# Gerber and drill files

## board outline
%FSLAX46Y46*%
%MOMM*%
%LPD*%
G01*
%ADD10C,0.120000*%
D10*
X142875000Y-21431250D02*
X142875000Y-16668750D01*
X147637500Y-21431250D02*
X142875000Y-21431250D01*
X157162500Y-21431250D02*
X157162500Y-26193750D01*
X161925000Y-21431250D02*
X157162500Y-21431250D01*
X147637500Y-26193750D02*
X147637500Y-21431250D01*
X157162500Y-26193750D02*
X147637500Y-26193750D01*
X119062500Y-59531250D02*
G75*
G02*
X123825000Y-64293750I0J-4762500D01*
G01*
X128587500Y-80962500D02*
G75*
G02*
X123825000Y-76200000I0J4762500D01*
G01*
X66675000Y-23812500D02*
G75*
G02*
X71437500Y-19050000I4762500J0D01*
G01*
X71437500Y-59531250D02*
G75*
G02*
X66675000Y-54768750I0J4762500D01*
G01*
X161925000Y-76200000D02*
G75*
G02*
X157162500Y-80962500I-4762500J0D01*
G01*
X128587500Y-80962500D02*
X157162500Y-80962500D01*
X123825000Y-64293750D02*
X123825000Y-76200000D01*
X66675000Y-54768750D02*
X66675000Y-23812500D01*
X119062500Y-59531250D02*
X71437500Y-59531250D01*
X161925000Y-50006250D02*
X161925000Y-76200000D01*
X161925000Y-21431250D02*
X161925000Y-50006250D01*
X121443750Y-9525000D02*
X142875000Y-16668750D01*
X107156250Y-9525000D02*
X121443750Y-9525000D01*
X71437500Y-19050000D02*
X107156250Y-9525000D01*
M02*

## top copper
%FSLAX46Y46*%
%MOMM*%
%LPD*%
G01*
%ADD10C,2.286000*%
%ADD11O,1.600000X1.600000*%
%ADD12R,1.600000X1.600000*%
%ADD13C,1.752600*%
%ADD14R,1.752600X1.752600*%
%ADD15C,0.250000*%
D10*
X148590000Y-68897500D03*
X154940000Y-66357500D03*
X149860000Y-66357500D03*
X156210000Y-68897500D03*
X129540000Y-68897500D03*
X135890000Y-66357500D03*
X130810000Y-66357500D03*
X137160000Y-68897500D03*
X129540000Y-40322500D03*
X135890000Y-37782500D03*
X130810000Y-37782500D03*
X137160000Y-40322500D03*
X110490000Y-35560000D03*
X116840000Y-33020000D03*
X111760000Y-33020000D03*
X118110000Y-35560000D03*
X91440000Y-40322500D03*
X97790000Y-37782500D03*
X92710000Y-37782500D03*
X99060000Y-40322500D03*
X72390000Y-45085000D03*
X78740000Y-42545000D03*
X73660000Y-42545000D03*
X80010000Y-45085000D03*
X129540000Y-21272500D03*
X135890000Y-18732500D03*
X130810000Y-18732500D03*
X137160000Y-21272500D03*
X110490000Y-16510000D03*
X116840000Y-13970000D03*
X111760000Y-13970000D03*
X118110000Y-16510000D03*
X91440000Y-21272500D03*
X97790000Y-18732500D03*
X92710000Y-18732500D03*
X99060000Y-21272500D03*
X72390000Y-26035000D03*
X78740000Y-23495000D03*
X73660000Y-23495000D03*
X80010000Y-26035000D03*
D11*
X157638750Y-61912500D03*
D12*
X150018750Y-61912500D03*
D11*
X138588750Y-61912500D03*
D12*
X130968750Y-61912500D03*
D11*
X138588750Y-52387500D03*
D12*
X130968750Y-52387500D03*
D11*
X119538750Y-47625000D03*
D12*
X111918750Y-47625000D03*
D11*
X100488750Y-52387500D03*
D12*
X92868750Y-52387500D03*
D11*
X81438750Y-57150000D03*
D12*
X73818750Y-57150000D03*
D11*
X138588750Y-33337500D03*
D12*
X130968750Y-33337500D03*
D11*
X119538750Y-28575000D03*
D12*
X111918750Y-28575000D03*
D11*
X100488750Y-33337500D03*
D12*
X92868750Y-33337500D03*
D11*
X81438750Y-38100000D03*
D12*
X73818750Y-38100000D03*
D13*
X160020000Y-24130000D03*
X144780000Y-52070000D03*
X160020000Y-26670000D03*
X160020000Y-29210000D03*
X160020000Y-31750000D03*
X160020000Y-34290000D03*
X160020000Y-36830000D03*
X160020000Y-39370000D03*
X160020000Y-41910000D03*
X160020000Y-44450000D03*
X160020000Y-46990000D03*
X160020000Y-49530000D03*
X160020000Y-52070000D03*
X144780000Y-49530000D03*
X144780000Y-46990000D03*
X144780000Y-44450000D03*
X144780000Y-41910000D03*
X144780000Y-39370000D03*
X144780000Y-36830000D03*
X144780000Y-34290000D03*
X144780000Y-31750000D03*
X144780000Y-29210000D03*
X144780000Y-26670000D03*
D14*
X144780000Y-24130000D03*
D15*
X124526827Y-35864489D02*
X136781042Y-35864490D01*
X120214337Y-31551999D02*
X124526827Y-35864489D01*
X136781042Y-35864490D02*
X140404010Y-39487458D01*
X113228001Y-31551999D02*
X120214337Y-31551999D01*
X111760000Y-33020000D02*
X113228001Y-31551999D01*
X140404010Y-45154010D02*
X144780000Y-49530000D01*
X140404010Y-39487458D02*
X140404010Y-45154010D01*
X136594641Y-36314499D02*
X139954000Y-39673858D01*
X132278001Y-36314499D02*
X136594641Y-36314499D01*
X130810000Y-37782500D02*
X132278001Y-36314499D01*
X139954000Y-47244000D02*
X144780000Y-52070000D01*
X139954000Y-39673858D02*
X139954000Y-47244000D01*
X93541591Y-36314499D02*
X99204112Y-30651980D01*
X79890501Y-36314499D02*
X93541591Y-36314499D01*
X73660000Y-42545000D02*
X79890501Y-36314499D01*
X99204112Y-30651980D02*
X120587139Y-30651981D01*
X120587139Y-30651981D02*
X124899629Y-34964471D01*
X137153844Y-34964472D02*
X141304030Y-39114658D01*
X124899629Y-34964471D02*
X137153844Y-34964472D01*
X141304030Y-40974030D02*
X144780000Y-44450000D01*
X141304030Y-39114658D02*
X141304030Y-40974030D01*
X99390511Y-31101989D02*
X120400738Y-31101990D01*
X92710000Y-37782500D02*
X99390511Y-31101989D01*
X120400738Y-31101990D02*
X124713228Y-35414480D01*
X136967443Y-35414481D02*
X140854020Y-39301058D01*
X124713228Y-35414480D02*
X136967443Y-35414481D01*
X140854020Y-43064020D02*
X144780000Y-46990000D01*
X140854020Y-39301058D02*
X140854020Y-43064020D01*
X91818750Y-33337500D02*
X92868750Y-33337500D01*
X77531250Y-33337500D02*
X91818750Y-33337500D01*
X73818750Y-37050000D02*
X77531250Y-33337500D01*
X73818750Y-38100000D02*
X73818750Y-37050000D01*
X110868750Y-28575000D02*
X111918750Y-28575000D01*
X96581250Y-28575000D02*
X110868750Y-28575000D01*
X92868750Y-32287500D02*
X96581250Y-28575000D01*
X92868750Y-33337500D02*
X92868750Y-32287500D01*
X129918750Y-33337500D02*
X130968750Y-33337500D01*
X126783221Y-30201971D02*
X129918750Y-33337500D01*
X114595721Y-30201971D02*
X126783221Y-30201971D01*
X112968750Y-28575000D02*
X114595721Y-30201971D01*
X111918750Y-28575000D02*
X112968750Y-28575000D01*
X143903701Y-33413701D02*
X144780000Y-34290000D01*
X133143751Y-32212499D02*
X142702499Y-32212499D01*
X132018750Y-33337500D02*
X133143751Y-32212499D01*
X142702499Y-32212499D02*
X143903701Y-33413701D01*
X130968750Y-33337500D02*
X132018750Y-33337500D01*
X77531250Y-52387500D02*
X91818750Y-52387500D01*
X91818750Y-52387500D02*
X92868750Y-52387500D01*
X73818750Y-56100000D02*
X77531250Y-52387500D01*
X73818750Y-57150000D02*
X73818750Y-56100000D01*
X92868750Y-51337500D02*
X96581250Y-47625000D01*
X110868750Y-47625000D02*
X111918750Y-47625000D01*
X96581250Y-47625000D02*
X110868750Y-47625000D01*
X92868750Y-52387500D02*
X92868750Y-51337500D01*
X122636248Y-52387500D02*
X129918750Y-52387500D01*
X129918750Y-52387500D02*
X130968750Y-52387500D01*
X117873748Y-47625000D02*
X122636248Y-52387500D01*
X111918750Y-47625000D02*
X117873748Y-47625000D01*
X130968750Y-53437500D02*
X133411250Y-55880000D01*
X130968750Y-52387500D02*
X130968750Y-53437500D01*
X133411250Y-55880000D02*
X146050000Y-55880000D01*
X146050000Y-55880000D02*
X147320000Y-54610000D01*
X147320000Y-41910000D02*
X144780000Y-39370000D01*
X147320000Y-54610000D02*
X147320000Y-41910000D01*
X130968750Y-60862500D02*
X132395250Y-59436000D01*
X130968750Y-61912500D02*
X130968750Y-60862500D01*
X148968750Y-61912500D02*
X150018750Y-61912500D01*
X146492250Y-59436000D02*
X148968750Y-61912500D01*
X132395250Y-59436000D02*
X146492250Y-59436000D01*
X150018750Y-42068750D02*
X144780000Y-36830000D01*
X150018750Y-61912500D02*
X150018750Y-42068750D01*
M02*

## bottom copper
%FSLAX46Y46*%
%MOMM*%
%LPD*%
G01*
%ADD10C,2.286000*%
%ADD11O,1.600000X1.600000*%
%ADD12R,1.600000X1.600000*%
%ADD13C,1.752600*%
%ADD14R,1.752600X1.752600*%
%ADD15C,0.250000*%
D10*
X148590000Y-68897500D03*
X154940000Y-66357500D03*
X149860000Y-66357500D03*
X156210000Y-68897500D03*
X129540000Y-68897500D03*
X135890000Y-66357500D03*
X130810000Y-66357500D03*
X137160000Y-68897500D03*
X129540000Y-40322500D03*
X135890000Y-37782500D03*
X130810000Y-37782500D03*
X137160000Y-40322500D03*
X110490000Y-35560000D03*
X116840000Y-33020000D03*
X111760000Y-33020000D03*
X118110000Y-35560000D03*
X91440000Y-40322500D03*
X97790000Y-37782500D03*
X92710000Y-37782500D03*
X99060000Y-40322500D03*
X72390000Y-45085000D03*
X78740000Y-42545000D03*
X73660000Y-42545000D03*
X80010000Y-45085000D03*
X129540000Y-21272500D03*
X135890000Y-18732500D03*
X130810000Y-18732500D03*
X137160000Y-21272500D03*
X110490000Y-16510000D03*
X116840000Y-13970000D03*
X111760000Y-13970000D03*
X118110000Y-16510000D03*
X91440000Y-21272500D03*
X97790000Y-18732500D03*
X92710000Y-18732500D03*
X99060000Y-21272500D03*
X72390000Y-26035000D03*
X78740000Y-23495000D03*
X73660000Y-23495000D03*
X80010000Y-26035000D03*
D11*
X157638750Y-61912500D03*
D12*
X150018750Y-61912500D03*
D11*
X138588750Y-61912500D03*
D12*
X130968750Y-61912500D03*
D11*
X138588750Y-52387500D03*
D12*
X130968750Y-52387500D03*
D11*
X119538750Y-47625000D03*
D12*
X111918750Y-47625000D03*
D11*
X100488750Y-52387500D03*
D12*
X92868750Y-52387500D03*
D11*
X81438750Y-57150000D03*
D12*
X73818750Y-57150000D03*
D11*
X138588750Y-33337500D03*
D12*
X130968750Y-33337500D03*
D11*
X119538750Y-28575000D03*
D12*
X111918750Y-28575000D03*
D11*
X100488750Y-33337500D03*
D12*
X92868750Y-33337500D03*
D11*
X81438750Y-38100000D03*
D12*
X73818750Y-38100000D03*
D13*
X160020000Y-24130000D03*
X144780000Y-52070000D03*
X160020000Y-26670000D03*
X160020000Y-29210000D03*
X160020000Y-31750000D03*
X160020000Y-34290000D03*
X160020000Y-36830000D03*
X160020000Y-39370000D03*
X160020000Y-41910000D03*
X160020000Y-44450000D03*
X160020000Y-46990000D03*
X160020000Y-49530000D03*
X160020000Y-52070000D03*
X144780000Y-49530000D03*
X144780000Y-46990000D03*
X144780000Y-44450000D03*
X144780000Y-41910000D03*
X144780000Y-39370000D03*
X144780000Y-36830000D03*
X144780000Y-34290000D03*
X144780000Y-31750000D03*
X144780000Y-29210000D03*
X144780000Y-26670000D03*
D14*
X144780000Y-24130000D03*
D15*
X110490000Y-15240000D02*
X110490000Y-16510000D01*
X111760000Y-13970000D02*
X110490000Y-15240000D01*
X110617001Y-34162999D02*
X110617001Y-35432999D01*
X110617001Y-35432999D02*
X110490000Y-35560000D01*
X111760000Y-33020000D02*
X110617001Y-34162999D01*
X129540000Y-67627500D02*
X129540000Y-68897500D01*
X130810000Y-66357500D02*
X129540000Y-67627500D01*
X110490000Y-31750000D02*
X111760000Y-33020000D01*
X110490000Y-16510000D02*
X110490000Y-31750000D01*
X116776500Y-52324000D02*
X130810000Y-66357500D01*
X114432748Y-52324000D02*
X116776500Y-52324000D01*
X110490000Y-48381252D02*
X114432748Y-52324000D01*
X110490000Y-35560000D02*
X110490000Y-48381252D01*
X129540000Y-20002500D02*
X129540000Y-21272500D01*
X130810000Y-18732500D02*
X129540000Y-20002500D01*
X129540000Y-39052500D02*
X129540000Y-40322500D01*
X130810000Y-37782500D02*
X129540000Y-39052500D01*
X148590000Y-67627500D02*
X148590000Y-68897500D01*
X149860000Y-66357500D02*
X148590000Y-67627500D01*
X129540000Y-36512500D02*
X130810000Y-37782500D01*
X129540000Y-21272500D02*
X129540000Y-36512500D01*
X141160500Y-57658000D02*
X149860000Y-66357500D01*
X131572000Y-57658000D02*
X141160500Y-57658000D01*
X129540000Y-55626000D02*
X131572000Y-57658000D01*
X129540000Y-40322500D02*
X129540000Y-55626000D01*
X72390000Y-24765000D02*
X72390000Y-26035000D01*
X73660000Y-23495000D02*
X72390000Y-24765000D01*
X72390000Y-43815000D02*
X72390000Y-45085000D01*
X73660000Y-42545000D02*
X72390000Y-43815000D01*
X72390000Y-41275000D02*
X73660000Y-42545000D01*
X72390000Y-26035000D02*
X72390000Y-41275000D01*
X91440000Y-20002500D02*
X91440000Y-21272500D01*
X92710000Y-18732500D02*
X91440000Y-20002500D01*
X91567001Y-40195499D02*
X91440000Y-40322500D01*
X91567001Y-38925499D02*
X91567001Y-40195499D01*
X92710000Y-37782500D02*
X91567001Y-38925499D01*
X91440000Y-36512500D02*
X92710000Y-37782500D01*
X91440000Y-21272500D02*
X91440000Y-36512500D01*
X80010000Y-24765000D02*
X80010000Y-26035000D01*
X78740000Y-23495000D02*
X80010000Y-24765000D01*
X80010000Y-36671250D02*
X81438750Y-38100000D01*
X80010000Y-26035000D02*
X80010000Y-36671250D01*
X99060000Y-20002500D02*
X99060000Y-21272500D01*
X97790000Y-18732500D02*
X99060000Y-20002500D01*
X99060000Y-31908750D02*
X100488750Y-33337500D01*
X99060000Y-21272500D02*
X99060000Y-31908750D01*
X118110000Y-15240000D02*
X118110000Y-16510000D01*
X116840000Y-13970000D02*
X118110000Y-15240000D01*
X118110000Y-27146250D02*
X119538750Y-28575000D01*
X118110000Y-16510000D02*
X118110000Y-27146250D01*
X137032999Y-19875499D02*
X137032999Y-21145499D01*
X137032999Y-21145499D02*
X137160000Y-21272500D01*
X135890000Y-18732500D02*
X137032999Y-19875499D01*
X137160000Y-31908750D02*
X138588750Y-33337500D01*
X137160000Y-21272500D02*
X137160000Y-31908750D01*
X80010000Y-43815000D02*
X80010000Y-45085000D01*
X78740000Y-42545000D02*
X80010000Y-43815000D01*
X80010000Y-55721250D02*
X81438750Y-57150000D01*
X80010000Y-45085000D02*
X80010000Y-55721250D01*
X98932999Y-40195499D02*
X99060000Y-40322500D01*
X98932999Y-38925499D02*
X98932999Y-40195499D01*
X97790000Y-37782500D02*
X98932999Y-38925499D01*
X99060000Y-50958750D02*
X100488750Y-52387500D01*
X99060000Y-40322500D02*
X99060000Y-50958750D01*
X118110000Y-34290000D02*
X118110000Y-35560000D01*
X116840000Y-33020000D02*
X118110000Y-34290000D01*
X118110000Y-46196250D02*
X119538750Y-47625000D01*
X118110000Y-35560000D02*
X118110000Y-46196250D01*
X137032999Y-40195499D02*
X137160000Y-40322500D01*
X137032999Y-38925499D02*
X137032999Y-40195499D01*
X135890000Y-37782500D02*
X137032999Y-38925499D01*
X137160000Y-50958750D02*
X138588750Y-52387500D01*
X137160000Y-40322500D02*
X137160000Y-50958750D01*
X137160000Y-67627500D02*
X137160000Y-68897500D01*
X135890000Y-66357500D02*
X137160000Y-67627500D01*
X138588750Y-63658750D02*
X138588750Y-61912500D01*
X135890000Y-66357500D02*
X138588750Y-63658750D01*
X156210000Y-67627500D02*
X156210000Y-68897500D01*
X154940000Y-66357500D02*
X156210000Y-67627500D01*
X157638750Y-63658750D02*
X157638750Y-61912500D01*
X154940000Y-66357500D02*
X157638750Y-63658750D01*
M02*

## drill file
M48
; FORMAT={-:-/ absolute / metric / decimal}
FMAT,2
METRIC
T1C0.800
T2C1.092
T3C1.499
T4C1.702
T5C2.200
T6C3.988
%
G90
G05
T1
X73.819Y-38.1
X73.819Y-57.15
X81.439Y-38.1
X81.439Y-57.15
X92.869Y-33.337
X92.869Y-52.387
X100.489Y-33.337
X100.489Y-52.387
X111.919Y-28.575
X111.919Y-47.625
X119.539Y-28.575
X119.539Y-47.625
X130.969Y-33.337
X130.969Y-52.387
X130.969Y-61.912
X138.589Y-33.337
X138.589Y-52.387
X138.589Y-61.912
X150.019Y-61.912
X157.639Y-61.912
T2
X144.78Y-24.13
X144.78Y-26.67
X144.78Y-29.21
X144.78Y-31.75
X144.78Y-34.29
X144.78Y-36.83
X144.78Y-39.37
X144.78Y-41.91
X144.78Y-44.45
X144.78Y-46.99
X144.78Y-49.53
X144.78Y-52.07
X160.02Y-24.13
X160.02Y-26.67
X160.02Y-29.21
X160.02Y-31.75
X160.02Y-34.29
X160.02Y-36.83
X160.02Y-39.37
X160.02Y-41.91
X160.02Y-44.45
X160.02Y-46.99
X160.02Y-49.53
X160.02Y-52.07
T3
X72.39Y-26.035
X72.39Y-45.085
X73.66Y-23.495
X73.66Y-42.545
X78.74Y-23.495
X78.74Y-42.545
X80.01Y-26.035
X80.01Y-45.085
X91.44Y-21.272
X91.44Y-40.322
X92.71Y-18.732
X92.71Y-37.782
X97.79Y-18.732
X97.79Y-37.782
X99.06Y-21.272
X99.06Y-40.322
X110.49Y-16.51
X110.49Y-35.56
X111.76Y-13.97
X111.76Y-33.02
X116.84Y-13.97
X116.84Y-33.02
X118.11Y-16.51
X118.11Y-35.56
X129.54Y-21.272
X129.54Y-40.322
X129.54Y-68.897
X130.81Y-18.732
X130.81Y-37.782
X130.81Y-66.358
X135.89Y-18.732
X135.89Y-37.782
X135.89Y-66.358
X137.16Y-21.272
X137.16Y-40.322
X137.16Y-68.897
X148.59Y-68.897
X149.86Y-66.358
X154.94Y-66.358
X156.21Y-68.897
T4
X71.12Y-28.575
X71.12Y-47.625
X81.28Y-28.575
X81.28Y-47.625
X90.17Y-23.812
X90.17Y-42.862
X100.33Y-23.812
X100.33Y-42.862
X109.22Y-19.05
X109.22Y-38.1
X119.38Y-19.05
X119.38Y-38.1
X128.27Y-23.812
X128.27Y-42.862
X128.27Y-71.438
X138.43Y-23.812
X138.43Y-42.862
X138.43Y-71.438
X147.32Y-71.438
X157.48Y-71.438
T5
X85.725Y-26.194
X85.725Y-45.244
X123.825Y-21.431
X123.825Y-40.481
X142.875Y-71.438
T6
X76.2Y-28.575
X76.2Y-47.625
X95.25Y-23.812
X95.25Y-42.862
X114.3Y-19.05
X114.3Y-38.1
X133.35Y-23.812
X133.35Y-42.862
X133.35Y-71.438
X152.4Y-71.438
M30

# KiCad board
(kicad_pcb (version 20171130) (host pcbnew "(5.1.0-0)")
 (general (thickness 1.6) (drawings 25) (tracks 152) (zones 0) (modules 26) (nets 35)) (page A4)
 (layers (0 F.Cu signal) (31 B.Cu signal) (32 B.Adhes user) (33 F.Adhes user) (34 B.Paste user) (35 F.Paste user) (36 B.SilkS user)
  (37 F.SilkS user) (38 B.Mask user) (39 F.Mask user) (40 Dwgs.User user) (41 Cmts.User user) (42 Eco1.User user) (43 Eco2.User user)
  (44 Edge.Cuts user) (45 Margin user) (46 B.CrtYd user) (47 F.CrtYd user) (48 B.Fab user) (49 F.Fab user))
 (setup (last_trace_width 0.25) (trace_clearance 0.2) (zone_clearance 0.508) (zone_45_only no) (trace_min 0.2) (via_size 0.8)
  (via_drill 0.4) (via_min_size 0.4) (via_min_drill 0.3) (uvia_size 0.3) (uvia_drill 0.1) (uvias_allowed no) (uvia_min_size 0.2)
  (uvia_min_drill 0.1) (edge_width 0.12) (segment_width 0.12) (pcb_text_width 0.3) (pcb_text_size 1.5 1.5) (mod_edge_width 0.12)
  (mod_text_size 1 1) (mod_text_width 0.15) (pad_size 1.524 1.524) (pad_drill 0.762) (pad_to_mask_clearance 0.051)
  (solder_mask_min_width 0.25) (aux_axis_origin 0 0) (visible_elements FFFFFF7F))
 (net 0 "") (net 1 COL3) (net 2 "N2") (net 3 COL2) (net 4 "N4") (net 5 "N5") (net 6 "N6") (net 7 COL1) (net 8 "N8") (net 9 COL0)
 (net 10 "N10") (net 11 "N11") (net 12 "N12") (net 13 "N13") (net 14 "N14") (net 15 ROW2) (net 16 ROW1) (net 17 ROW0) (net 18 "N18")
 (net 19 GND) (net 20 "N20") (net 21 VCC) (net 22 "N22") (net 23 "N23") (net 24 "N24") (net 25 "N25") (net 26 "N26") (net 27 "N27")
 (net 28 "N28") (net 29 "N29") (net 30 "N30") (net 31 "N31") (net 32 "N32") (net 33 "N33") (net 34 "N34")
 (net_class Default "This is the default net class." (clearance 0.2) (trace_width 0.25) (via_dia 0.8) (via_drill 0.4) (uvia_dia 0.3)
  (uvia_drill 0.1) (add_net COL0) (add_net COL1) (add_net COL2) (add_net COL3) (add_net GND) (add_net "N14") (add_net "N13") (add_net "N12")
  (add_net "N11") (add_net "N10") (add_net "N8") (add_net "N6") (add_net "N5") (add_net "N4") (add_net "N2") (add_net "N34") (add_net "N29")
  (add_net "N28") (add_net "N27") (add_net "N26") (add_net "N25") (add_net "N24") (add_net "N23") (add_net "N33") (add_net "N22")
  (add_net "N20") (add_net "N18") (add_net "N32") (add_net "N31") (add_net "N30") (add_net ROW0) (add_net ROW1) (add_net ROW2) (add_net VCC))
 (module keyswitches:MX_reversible (layer F.Cu) (at 152.4 71.4375)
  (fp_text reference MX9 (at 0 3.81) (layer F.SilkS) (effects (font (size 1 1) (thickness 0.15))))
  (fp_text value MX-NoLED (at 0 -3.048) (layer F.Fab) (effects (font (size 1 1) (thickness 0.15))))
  (pad "" np_thru_hole circle (at -5.08 0) (size 1.7018 1.7018) (drill 1.7018) (layers *.Cu *.Mask))
  (pad "" np_thru_hole circle (at 5.08 0) (size 1.7018 1.7018) (drill 1.7018) (layers *.Cu *.Mask))
  (pad 1 thru_hole circle (at -3.81 -2.54) (size 2.286 2.286) (drill 1.4986) (layers *.Cu *.Mask) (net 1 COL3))
  (pad "" np_thru_hole circle (at 0 0) (size 3.9878 3.9878) (drill 3.9878) (layers *.Cu *.Mask))
  (pad 2 thru_hole circle (at 2.54 -5.08) (size 2.286 2.286) (drill 1.4986) (layers *.Cu *.Mask) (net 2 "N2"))
  (pad 1 thru_hole circle (at -2.54 -5.08) (size 2.286 2.286) (drill 1.4986) (layers *.Cu *.Mask) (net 1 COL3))
  (pad 2 thru_hole circle (at 3.81 -2.54) (size 2.286 2.286) (drill 1.4986) (layers *.Cu *.Mask) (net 2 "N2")))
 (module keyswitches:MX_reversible (layer F.Cu) (at 133.35 71.4375)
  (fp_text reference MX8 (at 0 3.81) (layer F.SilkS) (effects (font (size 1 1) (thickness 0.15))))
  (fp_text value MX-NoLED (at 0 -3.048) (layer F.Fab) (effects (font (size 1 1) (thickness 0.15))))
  (pad "" np_thru_hole circle (at -5.08 0) (size 1.7018 1.7018) (drill 1.7018) (layers *.Cu *.Mask))
  (pad "" np_thru_hole circle (at 5.08 0) (size 1.7018 1.7018) (drill 1.7018) (layers *.Cu *.Mask))
  (pad 1 thru_hole circle (at -3.81 -2.54) (size 2.286 2.286) (drill 1.4986) (layers *.Cu *.Mask) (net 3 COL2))
  (pad "" np_thru_hole circle (at 0 0) (size 3.9878 3.9878) (drill 3.9878) (layers *.Cu *.Mask))
  (pad 2 thru_hole circle (at 2.54 -5.08) (size 2.286 2.286) (drill 1.4986) (layers *.Cu *.Mask) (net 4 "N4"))
  (pad 1 thru_hole circle (at -2.54 -5.08) (size 2.286 2.286) (drill 1.4986) (layers *.Cu *.Mask) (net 3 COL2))
  (pad 2 thru_hole circle (at 3.81 -2.54) (size 2.286 2.286) (drill 1.4986) (layers *.Cu *.Mask) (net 4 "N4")))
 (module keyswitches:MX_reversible (layer F.Cu) (at 133.35 42.8625)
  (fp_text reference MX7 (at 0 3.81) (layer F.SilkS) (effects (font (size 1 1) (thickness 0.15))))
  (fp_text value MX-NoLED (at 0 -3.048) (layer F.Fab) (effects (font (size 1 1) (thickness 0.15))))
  (pad "" np_thru_hole circle (at -5.08 0) (size 1.7018 1.7018) (drill 1.7018) (layers *.Cu *.Mask))
  (pad "" np_thru_hole circle (at 5.08 0) (size 1.7018 1.7018) (drill 1.7018) (layers *.Cu *.Mask))
  (pad 1 thru_hole circle (at -3.81 -2.54) (size 2.286 2.286) (drill 1.4986) (layers *.Cu *.Mask) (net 1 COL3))
  (pad "" np_thru_hole circle (at 0 0) (size 3.9878 3.9878) (drill 3.9878) (layers *.Cu *.Mask))
  (pad 2 thru_hole circle (at 2.54 -5.08) (size 2.286 2.286) (drill 1.4986) (layers *.Cu *.Mask) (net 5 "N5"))
  (pad 1 thru_hole circle (at -2.54 -5.08) (size 2.286 2.286) (drill 1.4986) (layers *.Cu *.Mask) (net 1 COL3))
  (pad 2 thru_hole circle (at 3.81 -2.54) (size 2.286 2.286) (drill 1.4986) (layers *.Cu *.Mask) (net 5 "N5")))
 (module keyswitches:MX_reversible (layer F.Cu) (at 114.3 38.1)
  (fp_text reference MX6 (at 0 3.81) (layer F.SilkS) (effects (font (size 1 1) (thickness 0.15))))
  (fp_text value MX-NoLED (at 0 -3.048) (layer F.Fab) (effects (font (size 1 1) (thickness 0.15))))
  (pad "" np_thru_hole circle (at -5.08 0) (size 1.7018 1.7018) (drill 1.7018) (layers *.Cu *.Mask))
  (pad "" np_thru_hole circle (at 5.08 0) (size 1.7018 1.7018) (drill 1.7018) (layers *.Cu *.Mask))
  (pad 1 thru_hole circle (at -3.81 -2.54) (size 2.286 2.286) (drill 1.4986) (layers *.Cu *.Mask) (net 3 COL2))
  (pad "" np_thru_hole circle (at 0 0) (size 3.9878 3.9878) (drill 3.9878) (layers *.Cu *.Mask))
  (pad 2 thru_hole circle (at 2.54 -5.08) (size 2.286 2.286) (drill 1.4986) (layers *.Cu *.Mask) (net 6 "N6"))
  (pad 1 thru_hole circle (at -2.54 -5.08) (size 2.286 2.286) (drill 1.4986) (layers *.Cu *.Mask) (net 3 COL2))
  (pad 2 thru_hole circle (at 3.81 -2.54) (size 2.286 2.286) (drill 1.4986) (layers *.Cu *.Mask) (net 6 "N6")))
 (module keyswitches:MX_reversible (layer F.Cu) (at 95.25 42.8625)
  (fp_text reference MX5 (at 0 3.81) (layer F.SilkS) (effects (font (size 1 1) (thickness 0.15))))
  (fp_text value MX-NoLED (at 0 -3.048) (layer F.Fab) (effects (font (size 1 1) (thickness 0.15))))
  (pad "" np_thru_hole circle (at -5.08 0) (size 1.7018 1.7018) (drill 1.7018) (layers *.Cu *.Mask))
  (pad "" np_thru_hole circle (at 5.08 0) (size 1.7018 1.7018) (drill 1.7018) (layers *.Cu *.Mask))
  (pad 1 thru_hole circle (at -3.81 -2.54) (size 2.286 2.286) (drill 1.4986) (layers *.Cu *.Mask) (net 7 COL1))
  (pad "" np_thru_hole circle (at 0 0) (size 3.9878 3.9878) (drill 3.9878) (layers *.Cu *.Mask))
  (pad 2 thru_hole circle (at 2.54 -5.08) (size 2.286 2.286) (drill 1.4986) (layers *.Cu *.Mask) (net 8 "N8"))
  (pad 1 thru_hole circle (at -2.54 -5.08) (size 2.286 2.286) (drill 1.4986) (layers *.Cu *.Mask) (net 7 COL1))
  (pad 2 thru_hole circle (at 3.81 -2.54) (size 2.286 2.286) (drill 1.4986) (layers *.Cu *.Mask) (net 8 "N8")))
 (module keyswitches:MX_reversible (layer F.Cu) (at 76.2 47.625)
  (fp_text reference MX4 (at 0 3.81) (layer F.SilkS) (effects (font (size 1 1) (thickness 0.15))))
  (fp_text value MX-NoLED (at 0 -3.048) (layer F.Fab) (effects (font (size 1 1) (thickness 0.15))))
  (pad "" np_thru_hole circle (at -5.08 0) (size 1.7018 1.7018) (drill 1.7018) (layers *.Cu *.Mask))
  (pad "" np_thru_hole circle (at 5.08 0) (size 1.7018 1.7018) (drill 1.7018) (layers *.Cu *.Mask))
  (pad 1 thru_hole circle (at -3.81 -2.54) (size 2.286 2.286) (drill 1.4986) (layers *.Cu *.Mask) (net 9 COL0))
  (pad "" np_thru_hole circle (at 0 0) (size 3.9878 3.9878) (drill 3.9878) (layers *.Cu *.Mask))
  (pad 2 thru_hole circle (at 2.54 -5.08) (size 2.286 2.286) (drill 1.4986) (layers *.Cu *.Mask) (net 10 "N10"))
  (pad 1 thru_hole circle (at -2.54 -5.08) (size 2.286 2.286) (drill 1.4986) (layers *.Cu *.Mask) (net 9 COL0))
  (pad 2 thru_hole circle (at 3.81 -2.54) (size 2.286 2.286) (drill 1.4986) (layers *.Cu *.Mask) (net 10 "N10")))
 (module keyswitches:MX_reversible (layer F.Cu) (at 133.35 23.8125)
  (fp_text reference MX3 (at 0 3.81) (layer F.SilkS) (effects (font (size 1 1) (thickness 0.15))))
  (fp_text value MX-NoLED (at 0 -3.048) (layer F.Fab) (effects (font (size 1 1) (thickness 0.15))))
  (pad "" np_thru_hole circle (at -5.08 0) (size 1.7018 1.7018) (drill 1.7018) (layers *.Cu *.Mask))
  (pad "" np_thru_hole circle (at 5.08 0) (size 1.7018 1.7018) (drill 1.7018) (layers *.Cu *.Mask))
  (pad 1 thru_hole circle (at -3.81 -2.54) (size 2.286 2.286) (drill 1.4986) (layers *.Cu *.Mask) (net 1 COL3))
  (pad "" np_thru_hole circle (at 0 0) (size 3.9878 3.9878) (drill 3.9878) (layers *.Cu *.Mask))
  (pad 2 thru_hole circle (at 2.54 -5.08) (size 2.286 2.286) (drill 1.4986) (layers *.Cu *.Mask) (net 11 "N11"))
  (pad 1 thru_hole circle (at -2.54 -5.08) (size 2.286 2.286) (drill 1.4986) (layers *.Cu *.Mask) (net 1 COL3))
  (pad 2 thru_hole circle (at 3.81 -2.54) (size 2.286 2.286) (drill 1.4986) (layers *.Cu *.Mask) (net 11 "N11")))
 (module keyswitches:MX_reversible (layer F.Cu) (at 114.3 19.05)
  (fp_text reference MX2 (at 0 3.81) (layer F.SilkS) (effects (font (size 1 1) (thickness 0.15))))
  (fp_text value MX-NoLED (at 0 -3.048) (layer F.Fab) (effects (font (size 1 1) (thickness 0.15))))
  (pad "" np_thru_hole circle (at -5.08 0) (size 1.7018 1.7018) (drill 1.7018) (layers *.Cu *.Mask))
  (pad "" np_thru_hole circle (at 5.08 0) (size 1.7018 1.7018) (drill 1.7018) (layers *.Cu *.Mask))
  (pad 1 thru_hole circle (at -3.81 -2.54) (size 2.286 2.286) (drill 1.4986) (layers *.Cu *.Mask) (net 3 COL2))
  (pad "" np_thru_hole circle (at 0 0) (size 3.9878 3.9878) (drill 3.9878) (layers *.Cu *.Mask))
  (pad 2 thru_hole circle (at 2.54 -5.08) (size 2.286 2.286) (drill 1.4986) (layers *.Cu *.Mask) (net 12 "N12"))
  (pad 1 thru_hole circle (at -2.54 -5.08) (size 2.286 2.286) (drill 1.4986) (layers *.Cu *.Mask) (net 3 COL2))
  (pad 2 thru_hole circle (at 3.81 -2.54) (size 2.286 2.286) (drill 1.4986) (layers *.Cu *.Mask) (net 12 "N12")))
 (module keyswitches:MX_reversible (layer F.Cu) (at 95.25 23.8125)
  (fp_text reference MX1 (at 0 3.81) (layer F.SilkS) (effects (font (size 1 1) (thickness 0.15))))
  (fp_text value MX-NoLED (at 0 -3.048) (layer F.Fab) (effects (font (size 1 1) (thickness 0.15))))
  (pad "" np_thru_hole circle (at -5.08 0) (size 1.7018 1.7018) (drill 1.7018) (layers *.Cu *.Mask))
  (pad "" np_thru_hole circle (at 5.08 0) (size 1.7018 1.7018) (drill 1.7018) (layers *.Cu *.Mask))
  (pad 1 thru_hole circle (at -3.81 -2.54) (size 2.286 2.286) (drill 1.4986) (layers *.Cu *.Mask) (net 7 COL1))
  (pad "" np_thru_hole circle (at 0 0) (size 3.9878 3.9878) (drill 3.9878) (layers *.Cu *.Mask))
  (pad 2 thru_hole circle (at 2.54 -5.08) (size 2.286 2.286) (drill 1.4986) (layers *.Cu *.Mask) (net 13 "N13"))
  (pad 1 thru_hole circle (at -2.54 -5.08) (size 2.286 2.286) (drill 1.4986) (layers *.Cu *.Mask) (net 7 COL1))
  (pad 2 thru_hole circle (at 3.81 -2.54) (size 2.286 2.286) (drill 1.4986) (layers *.Cu *.Mask) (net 13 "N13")))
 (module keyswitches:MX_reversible (layer F.Cu) (at 76.2 28.575)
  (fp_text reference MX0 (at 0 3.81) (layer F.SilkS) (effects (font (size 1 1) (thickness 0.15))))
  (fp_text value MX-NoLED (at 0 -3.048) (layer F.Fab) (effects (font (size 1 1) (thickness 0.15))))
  (pad "" np_thru_hole circle (at -5.08 0) (size 1.7018 1.7018) (drill 1.7018) (layers *.Cu *.Mask))
  (pad "" np_thru_hole circle (at 5.08 0) (size 1.7018 1.7018) (drill 1.7018) (layers *.Cu *.Mask))
  (pad 1 thru_hole circle (at -3.81 -2.54) (size 2.286 2.286) (drill 1.4986) (layers *.Cu *.Mask) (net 9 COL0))
  (pad "" np_thru_hole circle (at 0 0) (size 3.9878 3.9878) (drill 3.9878) (layers *.Cu *.Mask))
  (pad 2 thru_hole circle (at 2.54 -5.08) (size 2.286 2.286) (drill 1.4986) (layers *.Cu *.Mask) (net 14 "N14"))
  (pad 1 thru_hole circle (at -2.54 -5.08) (size 2.286 2.286) (drill 1.4986) (layers *.Cu *.Mask) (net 9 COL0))
  (pad 2 thru_hole circle (at 3.81 -2.54) (size 2.286 2.286) (drill 1.4986) (layers *.Cu *.Mask) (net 14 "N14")))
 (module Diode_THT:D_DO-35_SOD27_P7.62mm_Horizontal (layer F.Cu) (at 150.01875 61.9125)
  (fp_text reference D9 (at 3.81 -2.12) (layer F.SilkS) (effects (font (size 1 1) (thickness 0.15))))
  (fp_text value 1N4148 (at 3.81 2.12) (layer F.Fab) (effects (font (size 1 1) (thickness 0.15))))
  (pad 2 thru_hole oval (at 7.62 0) (size 1.6 1.6) (drill 0.8) (layers *.Cu *.Mask) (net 2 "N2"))
  (pad 1 thru_hole rect (at 0 0) (size 1.6 1.6) (drill 0.8) (layers *.Cu *.Mask) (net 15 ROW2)))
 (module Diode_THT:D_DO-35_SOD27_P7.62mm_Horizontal (layer F.Cu) (at 130.96875 61.9125)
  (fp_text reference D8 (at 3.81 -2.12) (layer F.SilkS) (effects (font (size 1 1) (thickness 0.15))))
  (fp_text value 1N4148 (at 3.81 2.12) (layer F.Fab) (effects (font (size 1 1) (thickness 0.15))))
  (pad 2 thru_hole oval (at 7.62 0) (size 1.6 1.6) (drill 0.8) (layers *.Cu *.Mask) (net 4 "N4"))
  (pad 1 thru_hole rect (at 0 0) (size 1.6 1.6) (drill 0.8) (layers *.Cu *.Mask) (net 15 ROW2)))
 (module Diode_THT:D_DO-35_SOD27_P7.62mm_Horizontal (layer F.Cu) (at 130.96875 52.3875)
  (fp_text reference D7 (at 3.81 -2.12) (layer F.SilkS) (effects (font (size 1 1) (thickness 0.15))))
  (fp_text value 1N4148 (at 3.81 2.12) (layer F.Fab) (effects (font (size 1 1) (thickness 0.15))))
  (pad 2 thru_hole oval (at 7.62 0) (size 1.6 1.6) (drill 0.8) (layers *.Cu *.Mask) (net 5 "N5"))
  (pad 1 thru_hole rect (at 0 0) (size 1.6 1.6) (drill 0.8) (layers *.Cu *.Mask) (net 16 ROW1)))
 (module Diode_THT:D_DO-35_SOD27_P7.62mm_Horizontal (layer F.Cu) (at 111.91875 47.625)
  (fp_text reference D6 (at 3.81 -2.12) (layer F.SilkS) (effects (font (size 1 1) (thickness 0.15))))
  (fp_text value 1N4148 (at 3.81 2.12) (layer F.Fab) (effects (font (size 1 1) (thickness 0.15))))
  (pad 2 thru_hole oval (at 7.62 0) (size 1.6 1.6) (drill 0.8) (layers *.Cu *.Mask) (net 6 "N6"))
  (pad 1 thru_hole rect (at 0 0) (size 1.6 1.6) (drill 0.8) (layers *.Cu *.Mask) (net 16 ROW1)))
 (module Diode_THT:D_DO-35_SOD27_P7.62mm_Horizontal (layer F.Cu) (at 92.86875 52.3875)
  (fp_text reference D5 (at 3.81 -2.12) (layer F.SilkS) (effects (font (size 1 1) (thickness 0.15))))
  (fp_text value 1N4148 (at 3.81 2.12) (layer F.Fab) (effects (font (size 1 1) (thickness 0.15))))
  (pad 2 thru_hole oval (at 7.62 0) (size 1.6 1.6) (drill 0.8) (layers *.Cu *.Mask) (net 8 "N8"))
  (pad 1 thru_hole rect (at 0 0) (size 1.6 1.6) (drill 0.8) (layers *.Cu *.Mask) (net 16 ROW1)))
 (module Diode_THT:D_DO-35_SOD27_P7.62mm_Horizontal (layer F.Cu) (at 73.81875 57.15)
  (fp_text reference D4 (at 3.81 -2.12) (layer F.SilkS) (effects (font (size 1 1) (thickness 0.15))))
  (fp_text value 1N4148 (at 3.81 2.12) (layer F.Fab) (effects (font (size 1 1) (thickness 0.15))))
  (pad 2 thru_hole oval (at 7.62 0) (size 1.6 1.6) (drill 0.8) (layers *.Cu *.Mask) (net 10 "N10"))
  (pad 1 thru_hole rect (at 0 0) (size 1.6 1.6) (drill 0.8) (layers *.Cu *.Mask) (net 16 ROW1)))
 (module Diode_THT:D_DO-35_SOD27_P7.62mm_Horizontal (layer F.Cu) (at 130.96875 33.3375)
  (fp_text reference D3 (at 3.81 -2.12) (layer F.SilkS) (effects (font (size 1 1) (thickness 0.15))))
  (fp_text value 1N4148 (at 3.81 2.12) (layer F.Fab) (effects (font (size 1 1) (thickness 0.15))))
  (pad 2 thru_hole oval (at 7.62 0) (size 1.6 1.6) (drill 0.8) (layers *.Cu *.Mask) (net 11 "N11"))
  (pad 1 thru_hole rect (at 0 0) (size 1.6 1.6) (drill 0.8) (layers *.Cu *.Mask) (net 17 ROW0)))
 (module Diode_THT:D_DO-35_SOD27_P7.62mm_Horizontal (layer F.Cu) (at 111.91875 28.575)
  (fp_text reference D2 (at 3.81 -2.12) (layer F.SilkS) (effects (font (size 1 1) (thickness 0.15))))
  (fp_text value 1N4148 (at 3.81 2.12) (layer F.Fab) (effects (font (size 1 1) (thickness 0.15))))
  (pad 2 thru_hole oval (at 7.62 0) (size 1.6 1.6) (drill 0.8) (layers *.Cu *.Mask) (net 12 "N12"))
  (pad 1 thru_hole rect (at 0 0) (size 1.6 1.6) (drill 0.8) (layers *.Cu *.Mask) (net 17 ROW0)))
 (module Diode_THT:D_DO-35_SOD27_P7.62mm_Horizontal (layer F.Cu) (at 92.86875 33.3375)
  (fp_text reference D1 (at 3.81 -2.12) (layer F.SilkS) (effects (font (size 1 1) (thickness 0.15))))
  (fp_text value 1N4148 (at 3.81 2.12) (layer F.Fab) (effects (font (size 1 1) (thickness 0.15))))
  (pad 2 thru_hole oval (at 7.62 0) (size 1.6 1.6) (drill 0.8) (layers *.Cu *.Mask) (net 13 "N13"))
  (pad 1 thru_hole rect (at 0 0) (size 1.6 1.6) (drill 0.8) (layers *.Cu *.Mask) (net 17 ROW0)))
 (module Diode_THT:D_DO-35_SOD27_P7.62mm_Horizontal (layer F.Cu) (at 73.81875 38.1)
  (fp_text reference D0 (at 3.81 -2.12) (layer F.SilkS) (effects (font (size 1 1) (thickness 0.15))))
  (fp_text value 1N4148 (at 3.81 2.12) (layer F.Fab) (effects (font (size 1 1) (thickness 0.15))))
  (pad 2 thru_hole oval (at 7.62 0) (size 1.6 1.6) (drill 0.8) (layers *.Cu *.Mask) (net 14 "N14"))
  (pad 1 thru_hole rect (at 0 0) (size 1.6 1.6) (drill 0.8) (layers *.Cu *.Mask) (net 17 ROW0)))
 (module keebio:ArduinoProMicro (layer F.Cu) (at 152.4 38.1 270)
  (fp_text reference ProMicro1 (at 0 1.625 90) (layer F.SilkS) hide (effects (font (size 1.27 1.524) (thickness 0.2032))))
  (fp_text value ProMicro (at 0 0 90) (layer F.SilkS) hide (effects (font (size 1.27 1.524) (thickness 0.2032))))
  (pad 24 thru_hole circle (at -13.97 -7.62 270) (size 1.7526 1.7526) (drill 1.0922) (layers *.Cu *.SilkS *.Mask) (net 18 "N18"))
  (pad 12 thru_hole circle (at 13.97 7.62 270) (size 1.7526 1.7526) (drill 1.0922) (layers *.Cu *.SilkS *.Mask) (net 1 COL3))
  (pad 23 thru_hole circle (at -11.43 -7.62 270) (size 1.7526 1.7526) (drill 1.0922) (layers *.Cu *.SilkS *.Mask) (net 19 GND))
  (pad 22 thru_hole circle (at -8.89 -7.62 270) (size 1.7526 1.7526) (drill 1.0922) (layers *.Cu *.SilkS *.Mask) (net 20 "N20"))
  (pad 21 thru_hole circle (at -6.35 -7.62 270) (size 1.7526 1.7526) (drill 1.0922) (layers *.Cu *.SilkS *.Mask) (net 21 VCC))
  (pad 20 thru_hole circle (at -3.81 -7.62 270) (size 1.7526 1.7526) (drill 1.0922) (layers *.Cu *.SilkS *.Mask) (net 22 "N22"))
  (pad 19 thru_hole circle (at -1.27 -7.62 270) (size 1.7526 1.7526) (drill 1.0922) (layers *.Cu *.SilkS *.Mask) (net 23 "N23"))
  (pad 18 thru_hole circle (at 1.27 -7.62 270) (size 1.7526 1.7526) (drill 1.0922) (layers *.Cu *.SilkS *.Mask) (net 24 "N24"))
  (pad 17 thru_hole circle (at 3.81 -7.62 270) (size 1.7526 1.7526) (drill 1.0922) (layers *.Cu *.SilkS *.Mask) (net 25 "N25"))
  (pad 16 thru_hole circle (at 6.35 -7.62 270) (size 1.7526 1.7526) (drill 1.0922) (layers *.Cu *.SilkS *.Mask) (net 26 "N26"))
  (pad 15 thru_hole circle (at 8.89 -7.62 270) (size 1.7526 1.7526) (drill 1.0922) (layers *.Cu *.SilkS *.Mask) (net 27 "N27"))
  (pad 14 thru_hole circle (at 11.43 -7.62 270) (size 1.7526 1.7526) (drill 1.0922) (layers *.Cu *.SilkS *.Mask) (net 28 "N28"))
  (pad 13 thru_hole circle (at 13.97 -7.62 270) (size 1.7526 1.7526) (drill 1.0922) (layers *.Cu *.SilkS *.Mask) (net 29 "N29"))
  (pad 11 thru_hole circle (at 11.43 7.62 270) (size 1.7526 1.7526) (drill 1.0922) (layers *.Cu *.SilkS *.Mask) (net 3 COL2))
  (pad 10 thru_hole circle (at 8.89 7.62 270) (size 1.7526 1.7526) (drill 1.0922) (layers *.Cu *.SilkS *.Mask) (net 7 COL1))
  (pad 9 thru_hole circle (at 6.35 7.62 270) (size 1.7526 1.7526) (drill 1.0922) (layers *.Cu *.SilkS *.Mask) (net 9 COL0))
  (pad 8 thru_hole circle (at 3.81 7.62 270) (size 1.7526 1.7526) (drill 1.0922) (layers *.Cu *.SilkS *.Mask) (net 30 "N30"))
  (pad 7 thru_hole circle (at 1.27 7.62 270) (size 1.7526 1.7526) (drill 1.0922) (layers *.Cu *.SilkS *.Mask) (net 16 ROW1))
  (pad 6 thru_hole circle (at -1.27 7.62 270) (size 1.7526 1.7526) (drill 1.0922) (layers *.Cu *.SilkS *.Mask) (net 15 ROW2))
  (pad 5 thru_hole circle (at -3.81 7.62 270) (size 1.7526 1.7526) (drill 1.0922) (layers *.Cu *.SilkS *.Mask) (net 17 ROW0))
  (pad 4 thru_hole circle (at -6.35 7.62 270) (size 1.7526 1.7526) (drill 1.0922) (layers *.Cu *.SilkS *.Mask) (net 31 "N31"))
  (pad 3 thru_hole circle (at -8.89 7.62 270) (size 1.7526 1.7526) (drill 1.0922) (layers *.Cu *.SilkS *.Mask) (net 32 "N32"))
  (pad 2 thru_hole circle (at -11.43 7.62 270) (size 1.7526 1.7526) (drill 1.0922) (layers *.Cu *.SilkS *.Mask) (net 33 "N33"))
  (pad 1 thru_hole rect (at -13.97 7.62 270) (size 1.7526 1.7526) (drill 1.0922) (layers *.Cu *.SilkS *.Mask) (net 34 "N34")))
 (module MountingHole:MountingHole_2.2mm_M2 (layer F.Cu) (at 85.725 45.24375)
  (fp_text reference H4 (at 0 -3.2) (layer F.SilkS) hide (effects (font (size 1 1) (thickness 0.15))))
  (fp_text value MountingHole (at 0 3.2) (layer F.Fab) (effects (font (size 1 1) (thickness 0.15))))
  (pad 1 np_thru_hole circle (at 0 0) (size 2.2 2.2) (drill 2.2) (layers *.Cu *.Mask)))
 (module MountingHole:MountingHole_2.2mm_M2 (layer F.Cu) (at 123.825 40.48125)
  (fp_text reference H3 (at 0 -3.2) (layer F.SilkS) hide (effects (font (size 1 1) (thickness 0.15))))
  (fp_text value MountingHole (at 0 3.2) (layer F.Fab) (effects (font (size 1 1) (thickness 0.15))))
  (pad 1 np_thru_hole circle (at 0 0) (size 2.2 2.2) (drill 2.2) (layers *.Cu *.Mask)))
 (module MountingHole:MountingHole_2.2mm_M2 (layer F.Cu) (at 142.875 71.4375)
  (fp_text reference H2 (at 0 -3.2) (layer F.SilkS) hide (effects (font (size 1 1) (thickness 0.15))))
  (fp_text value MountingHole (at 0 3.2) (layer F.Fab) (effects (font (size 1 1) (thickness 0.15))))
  (pad 1 np_thru_hole circle (at 0 0) (size 2.2 2.2) (drill 2.2) (layers *.Cu *.Mask)))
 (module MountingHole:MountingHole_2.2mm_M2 (layer F.Cu) (at 123.825 21.43125)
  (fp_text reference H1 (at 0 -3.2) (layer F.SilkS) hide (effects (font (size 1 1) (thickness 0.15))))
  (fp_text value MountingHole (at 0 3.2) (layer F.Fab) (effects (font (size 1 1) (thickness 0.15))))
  (pad 1 np_thru_hole circle (at 0 0) (size 2.2 2.2) (drill 2.2) (layers *.Cu *.Mask)))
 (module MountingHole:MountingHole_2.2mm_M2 (layer F.Cu) (at 85.725 26.19375)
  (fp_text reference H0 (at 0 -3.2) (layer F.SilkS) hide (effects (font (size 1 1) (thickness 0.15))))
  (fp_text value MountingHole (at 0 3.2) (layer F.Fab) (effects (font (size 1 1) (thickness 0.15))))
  (pad 1 np_thru_hole circle (at 0 0) (size 2.2 2.2) (drill 2.2) (layers *.Cu *.Mask)))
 (gr_line (start 142.875 21.43125) (end 142.875 16.66875) (layer Edge.Cuts) (width 0.12))
 (gr_line (start 147.6375 21.43125) (end 142.875 21.43125) (layer Edge.Cuts) (width 0.12))
 (gr_line (start 157.1625 21.43125) (end 157.1625 26.19375) (layer Edge.Cuts) (width 0.12))
 (gr_line (start 161.925 21.43125) (end 157.1625 21.43125) (layer Edge.Cuts) (width 0.12))
 (gr_line (start 147.6375 26.19375) (end 147.6375 21.43125) (layer Edge.Cuts) (width 0.12))
 (gr_line (start 157.1625 26.19375) (end 147.6375 26.19375) (layer Edge.Cuts) (width 0.12))
 (gr_arc (start 119.0625 64.29375) (end 123.825 64.29375) (angle -90) (layer Edge.Cuts) (width 0.12))
 (gr_arc (start 128.5875 76.2) (end 123.825 76.2) (angle -90) (layer Edge.Cuts) (width 0.12))
 (gr_arc (start 71.4375 23.8125) (end 71.4375 19.05) (angle -90) (layer Edge.Cuts) (width 0.12))
 (gr_arc (start 71.4375 54.76875) (end 66.675 54.76875) (angle -90) (layer Edge.Cuts) (width 0.12))
 (gr_arc (start 157.1625 76.2) (end 157.1625 80.9625) (angle -90) (layer Edge.Cuts) (width 0.12))
 (gr_line (start 128.5875 80.9625) (end 157.1625 80.9625) (layer Edge.Cuts) (width 0.12))
 (gr_line (start 123.825 64.29375) (end 123.825 76.2) (layer Edge.Cuts) (width 0.12))
 (gr_line (start 66.675 54.76875) (end 66.675 23.8125) (layer Edge.Cuts) (width 0.12))
 (gr_line (start 119.0625 59.53125) (end 71.4375 59.53125) (layer Edge.Cuts) (width 0.12))
 (gr_line (start 161.925 50.00625) (end 161.925 76.2) (layer Edge.Cuts) (width 0.12))
 (gr_line (start 161.925 21.43125) (end 161.925 50.00625) (layer Edge.Cuts) (width 0.12))
 (gr_line (start 121.44375 9.525) (end 142.875 16.66875) (layer Edge.Cuts) (width 0.12))
 (gr_line (start 107.15625 9.525) (end 121.44375 9.525) (layer Edge.Cuts) (width 0.12))
 (gr_line (start 71.4375 19.05) (end 107.15625 9.525) (layer Edge.Cuts) (width 0.12))
 (segment (start 110.49 15.24) (end 110.49 16.51) (width 0.25) (layer B.Cu) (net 3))
 (segment (start 111.76 13.97) (end 110.49 15.24) (width 0.25) (layer B.Cu) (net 3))
 (segment (start 110.617001 34.162999) (end 110.617001 35.432999) (width 0.25) (layer B.Cu) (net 3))
 (segment (start 110.617001 35.432999) (end 110.49 35.56) (width 0.25) (layer B.Cu) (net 3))
 (segment (start 111.76 33.02) (end 110.617001 34.162999) (width 0.25) (layer B.Cu) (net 3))
 (segment (start 129.54 67.6275) (end 129.54 68.8975) (width 0.25) (layer B.Cu) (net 3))
 (segment (start 130.81 66.3575) (end 129.54 67.6275) (width 0.25) (layer B.Cu) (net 3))
 (segment (start 110.49 31.75) (end 111.76 33.02) (width 0.25) (layer B.Cu) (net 3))
 (segment (start 110.49 16.51) (end 110.49 31.75) (width 0.25) (layer B.Cu) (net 3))
 (segment (start 124.526827 35.864489) (end 136.781042 35.86449) (width 0.25) (layer F.Cu) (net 3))
 (segment (start 120.214337 31.551999) (end 124.526827 35.864489) (width 0.25) (layer F.Cu) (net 3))
 (segment (start 136.781042 35.86449) (end 140.40401 39.487458) (width 0.25) (layer F.Cu) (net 3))
 (segment (start 113.228001 31.551999) (end 120.214337 31.551999) (width 0.25) (layer F.Cu) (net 3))
 (segment (start 111.76 33.02) (end 113.228001 31.551999) (width 0.25) (layer F.Cu) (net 3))
 (segment (start 140.40401 45.15401) (end 144.78 49.53) (width 0.25) (layer F.Cu) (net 3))
 (segment (start 140.40401 39.487458) (end 140.40401 45.15401) (width 0.25) (layer F.Cu) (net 3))
 (segment (start 116.7765 52.324) (end 130.81 66.3575) (width 0.25) (layer B.Cu) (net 3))
 (segment (start 114.432748 52.324) (end 116.7765 52.324) (width 0.25) (layer B.Cu) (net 3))
 (segment (start 110.49 48.381252) (end 114.432748 52.324) (width 0.25) (layer B.Cu) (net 3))
 (segment (start 110.49 35.56) (end 110.49 48.381252) (width 0.25) (layer B.Cu) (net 3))
 (segment (start 129.54 20.0025) (end 129.54 21.2725) (width 0.25) (layer B.Cu) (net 1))
 (segment (start 130.81 18.7325) (end 129.54 20.0025) (width 0.25) (layer B.Cu) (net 1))
 (segment (start 129.54 39.0525) (end 129.54 40.3225) (width 0.25) (layer B.Cu) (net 1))
 (segment (start 130.81 37.7825) (end 129.54 39.0525) (width 0.25) (layer B.Cu) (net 1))
 (segment (start 148.59 67.6275) (end 148.59 68.8975) (width 0.25) (layer B.Cu) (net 1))
 (segment (start 149.86 66.3575) (end 148.59 67.6275) (width 0.25) (layer B.Cu) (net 1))
 (segment (start 129.54 36.5125) (end 130.81 37.7825) (width 0.25) (layer B.Cu) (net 1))
 (segment (start 129.54 21.2725) (end 129.54 36.5125) (width 0.25) (layer B.Cu) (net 1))
 (segment (start 136.594641 36.314499) (end 139.954 39.673858) (width 0.25) (layer F.Cu) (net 1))
 (segment (start 132.278001 36.314499) (end 136.594641 36.314499) (width 0.25) (layer F.Cu) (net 1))
 (segment (start 130.81 37.7825) (end 132.278001 36.314499) (width 0.25) (layer F.Cu) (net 1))
 (segment (start 139.954 47.244) (end 144.78 52.07) (width 0.25) (layer F.Cu) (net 1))
 (segment (start 139.954 39.673858) (end 139.954 47.244) (width 0.25) (layer F.Cu) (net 1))
 (segment (start 141.1605 57.658) (end 149.86 66.3575) (width 0.25) (layer B.Cu) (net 1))
 (segment (start 131.572 57.658) (end 141.1605 57.658) (width 0.25) (layer B.Cu) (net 1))
 (segment (start 129.54 55.626) (end 131.572 57.658) (width 0.25) (layer B.Cu) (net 1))
 (segment (start 129.54 40.3225) (end 129.54 55.626) (width 0.25) (layer B.Cu) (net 1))
 (segment (start 72.39 24.765) (end 72.39 26.035) (width 0.25) (layer B.Cu) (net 9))
 (segment (start 73.66 23.495) (end 72.39 24.765) (width 0.25) (layer B.Cu) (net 9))
 (segment (start 72.39 43.815) (end 72.39 45.085) (width 0.25) (layer B.Cu) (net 9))
 (segment (start 73.66 42.545) (end 72.39 43.815) (width 0.25) (layer B.Cu) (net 9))
 (segment (start 72.39 41.275) (end 73.66 42.545) (width 0.25) (layer B.Cu) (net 9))
 (segment (start 72.39 26.035) (end 72.39 41.275) (width 0.25) (layer B.Cu) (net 9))
 (segment (start 93.541591 36.314499) (end 99.204112 30.65198) (width 0.25) (layer F.Cu) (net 9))
 (segment (start 79.890501 36.314499) (end 93.541591 36.314499) (width 0.25) (layer F.Cu) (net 9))
 (segment (start 73.66 42.545) (end 79.890501 36.314499) (width 0.25) (layer F.Cu) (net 9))
 (segment (start 99.204112 30.65198) (end 120.587139 30.651981) (width 0.25) (layer F.Cu) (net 9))
 (segment (start 120.587139 30.651981) (end 124.899629 34.964471) (width 0.25) (layer F.Cu) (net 9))
 (segment (start 137.153844 34.964472) (end 141.30403 39.114658) (width 0.25) (layer F.Cu) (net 9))
 (segment (start 124.899629 34.964471) (end 137.153844 34.964472) (width 0.25) (layer F.Cu) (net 9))
 (segment (start 141.30403 40.97403) (end 144.78 44.45) (width 0.25) (layer F.Cu) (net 9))
 (segment (start 141.30403 39.114658) (end 141.30403 40.97403) (width 0.25) (layer F.Cu) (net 9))
 (segment (start 91.44 20.0025) (end 91.44 21.2725) (width 0.25) (layer B.Cu) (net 7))
 (segment (start 92.71 18.7325) (end 91.44 20.0025) (width 0.25) (layer B.Cu) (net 7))
 (segment (start 91.567001 40.195499) (end 91.44 40.3225) (width 0.25) (layer B.Cu) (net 7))
 (segment (start 91.567001 38.925499) (end 91.567001 40.195499) (width 0.25) (layer B.Cu) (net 7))
 (segment (start 92.71 37.7825) (end 91.567001 38.925499) (width 0.25) (layer B.Cu) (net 7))
 (segment (start 91.44 36.5125) (end 92.71 37.7825) (width 0.25) (layer B.Cu) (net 7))
 (segment (start 91.44 21.2725) (end 91.44 36.5125) (width 0.25) (layer B.Cu) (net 7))
 (segment (start 99.390511 31.101989) (end 120.400738 31.10199) (width 0.25) (layer F.Cu) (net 7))
 (segment (start 92.71 37.7825) (end 99.390511 31.101989) (width 0.25) (layer F.Cu) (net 7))
 (segment (start 120.400738 31.10199) (end 124.713228 35.41448) (width 0.25) (layer F.Cu) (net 7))
 (segment (start 136.967443 35.414481) (end 140.85402 39.301058) (width 0.25) (layer F.Cu) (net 7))
 (segment (start 124.713228 35.41448) (end 136.967443 35.414481) (width 0.25) (layer F.Cu) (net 7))
 (segment (start 140.85402 43.06402) (end 144.78 46.99) (width 0.25) (layer F.Cu) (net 7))
 (segment (start 140.85402 39.301058) (end 140.85402 43.06402) (width 0.25) (layer F.Cu) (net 7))
 (segment (start 91.81875 33.3375) (end 92.86875 33.3375) (width 0.25) (layer F.Cu) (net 17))
 (segment (start 77.53125 33.3375) (end 91.81875 33.3375) (width 0.25) (layer F.Cu) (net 17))
 (segment (start 73.81875 37.05) (end 77.53125 33.3375) (width 0.25) (layer F.Cu) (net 17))
 (segment (start 73.81875 38.1) (end 73.81875 37.05) (width 0.25) (layer F.Cu) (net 17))
 (segment (start 110.86875 28.575) (end 111.91875 28.575) (width 0.25) (layer F.Cu) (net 17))
 (segment (start 96.58125 28.575) (end 110.86875 28.575) (width 0.25) (layer F.Cu) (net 17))
 (segment (start 92.86875 32.2875) (end 96.58125 28.575) (width 0.25) (layer F.Cu) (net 17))
 (segment (start 92.86875 33.3375) (end 92.86875 32.2875) (width 0.25) (layer F.Cu) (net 17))
 (segment (start 129.91875 33.3375) (end 130.96875 33.3375) (width 0.25) (layer F.Cu) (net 17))
 (segment (start 126.783221 30.201971) (end 129.91875 33.3375) (width 0.25) (layer F.Cu) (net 17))
 (segment (start 114.595721 30.201971) (end 126.783221 30.201971) (width 0.25) (layer F.Cu) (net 17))
 (segment (start 112.96875 28.575) (end 114.595721 30.201971) (width 0.25) (layer F.Cu) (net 17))
 (segment (start 111.91875 28.575) (end 112.96875 28.575) (width 0.25) (layer F.Cu) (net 17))
 (segment (start 143.903701 33.413701) (end 144.78 34.29) (width 0.25) (layer F.Cu) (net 17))
 (segment (start 133.143751 32.212499) (end 142.702499 32.212499) (width 0.25) (layer F.Cu) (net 17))
 (segment (start 132.01875 33.3375) (end 133.143751 32.212499) (width 0.25) (layer F.Cu) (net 17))
 (segment (start 142.702499 32.212499) (end 143.903701 33.413701) (width 0.25) (layer F.Cu) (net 17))
 (segment (start 130.96875 33.3375) (end 132.01875 33.3375) (width 0.25) (layer F.Cu) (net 17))
 (segment (start 77.53125 52.3875) (end 91.81875 52.3875) (width 0.25) (layer F.Cu) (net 16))
 (segment (start 91.81875 52.3875) (end 92.86875 52.3875) (width 0.25) (layer F.Cu) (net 16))
 (segment (start 73.81875 56.1) (end 77.53125 52.3875) (width 0.25) (layer F.Cu) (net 16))
 (segment (start 73.81875 57.15) (end 73.81875 56.1) (width 0.25) (layer F.Cu) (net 16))
 (segment (start 92.86875 51.3375) (end 96.58125 47.625) (width 0.25) (layer F.Cu) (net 16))
 (segment (start 110.86875 47.625) (end 111.91875 47.625) (width 0.25) (layer F.Cu) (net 16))
 (segment (start 96.58125 47.625) (end 110.86875 47.625) (width 0.25) (layer F.Cu) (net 16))
 (segment (start 92.86875 52.3875) (end 92.86875 51.3375) (width 0.25) (layer F.Cu) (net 16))
 (segment (start 122.636248 52.3875) (end 129.91875 52.3875) (width 0.25) (layer F.Cu) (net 16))
 (segment (start 129.91875 52.3875) (end 130.96875 52.3875) (width 0.25) (layer F.Cu) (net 16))
 (segment (start 117.873748 47.625) (end 122.636248 52.3875) (width 0.25) (layer F.Cu) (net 16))
 (segment (start 111.91875 47.625) (end 117.873748 47.625) (width 0.25) (layer F.Cu) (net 16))
 (segment (start 130.96875 53.4375) (end 133.41125 55.88) (width 0.25) (layer F.Cu) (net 16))
 (segment (start 130.96875 52.3875) (end 130.96875 53.4375) (width 0.25) (layer F.Cu) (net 16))
 (segment (start 133.41125 55.88) (end 146.05 55.88) (width 0.25) (layer F.Cu) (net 16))
 (segment (start 146.05 55.88) (end 147.32 54.61) (width 0.25) (layer F.Cu) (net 16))
 (segment (start 147.32 41.91) (end 144.78 39.37) (width 0.25) (layer F.Cu) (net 16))
 (segment (start 147.32 54.61) (end 147.32 41.91) (width 0.25) (layer F.Cu) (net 16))
 (segment (start 130.96875 60.8625) (end 132.39525 59.436) (width 0.25) (layer F.Cu) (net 15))
 (segment (start 130.96875 61.9125) (end 130.96875 60.8625) (width 0.25) (layer F.Cu) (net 15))
 (segment (start 148.96875 61.9125) (end 150.01875 61.9125) (width 0.25) (layer F.Cu) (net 15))
 (segment (start 146.49225 59.436) (end 148.96875 61.9125) (width 0.25) (layer F.Cu) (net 15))
 (segment (start 132.39525 59.436) (end 146.49225 59.436) (width 0.25) (layer F.Cu) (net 15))
 (segment (start 150.01875 42.06875) (end 144.78 36.83) (width 0.25) (layer F.Cu) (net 15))
 (segment (start 150.01875 61.9125) (end 150.01875 42.06875) (width 0.25) (layer F.Cu) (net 15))
 (segment (start 80.01 24.765) (end 80.01 26.035) (width 0.25) (layer B.Cu) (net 14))
 (segment (start 78.74 23.495) (end 80.01 24.765) (width 0.25) (layer B.Cu) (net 14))
 (segment (start 80.01 36.67125) (end 81.43875 38.1) (width 0.25) (layer B.Cu) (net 14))
 (segment (start 80.01 26.035) (end 80.01 36.67125) (width 0.25) (layer B.Cu) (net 14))
 (segment (start 99.06 20.0025) (end 99.06 21.2725) (width 0.25) (layer B.Cu) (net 13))
 (segment (start 97.79 18.7325) (end 99.06 20.0025) (width 0.25) (layer B.Cu) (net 13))
 (segment (start 99.06 31.90875) (end 100.48875 33.3375) (width 0.25) (layer B.Cu) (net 13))
 (segment (start 99.06 21.2725) (end 99.06 31.90875) (width 0.25) (layer B.Cu) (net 13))
 (segment (start 118.11 15.24) (end 118.11 16.51) (width 0.25) (layer B.Cu) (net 12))
 (segment (start 116.84 13.97) (end 118.11 15.24) (width 0.25) (layer B.Cu) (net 12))
 (segment (start 118.11 27.14625) (end 119.53875 28.575) (width 0.25) (layer B.Cu) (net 12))
 (segment (start 118.11 16.51) (end 118.11 27.14625) (width 0.25) (layer B.Cu) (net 12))
 (segment (start 137.032999 19.875499) (end 137.032999 21.145499) (width 0.25) (layer B.Cu) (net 11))
 (segment (start 137.032999 21.145499) (end 137.16 21.2725) (width 0.25) (layer B.Cu) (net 11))
 (segment (start 135.89 18.7325) (end 137.032999 19.875499) (width 0.25) (layer B.Cu) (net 11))
 (segment (start 137.16 31.90875) (end 138.58875 33.3375) (width 0.25) (layer B.Cu) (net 11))
 (segment (start 137.16 21.2725) (end 137.16 31.90875) (width 0.25) (layer B.Cu) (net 11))
 (segment (start 80.01 43.815) (end 80.01 45.085) (width 0.25) (layer B.Cu) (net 10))
 (segment (start 78.74 42.545) (end 80.01 43.815) (width 0.25) (layer B.Cu) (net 10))
 (segment (start 80.01 55.72125) (end 81.43875 57.15) (width 0.25) (layer B.Cu) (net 10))
 (segment (start 80.01 45.085) (end 80.01 55.72125) (width 0.25) (layer B.Cu) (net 10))
 (segment (start 98.932999 40.195499) (end 99.06 40.3225) (width 0.25) (layer B.Cu) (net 8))
 (segment (start 98.932999 38.925499) (end 98.932999 40.195499) (width 0.25) (layer B.Cu) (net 8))
 (segment (start 97.79 37.7825) (end 98.932999 38.925499) (width 0.25) (layer B.Cu) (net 8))
 (segment (start 99.06 50.95875) (end 100.48875 52.3875) (width 0.25) (layer B.Cu) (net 8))
 (segment (start 99.06 40.3225) (end 99.06 50.95875) (width 0.25) (layer B.Cu) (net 8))
 (segment (start 118.11 34.29) (end 118.11 35.56) (width 0.25) (layer B.Cu) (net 6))
 (segment (start 116.84 33.02) (end 118.11 34.29) (width 0.25) (layer B.Cu) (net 6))
 (segment (start 118.11 46.19625) (end 119.53875 47.625) (width 0.25) (layer B.Cu) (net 6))
 (segment (start 118.11 35.56) (end 118.11 46.19625) (width 0.25) (layer B.Cu) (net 6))
 (segment (start 137.032999 40.195499) (end 137.16 40.3225) (width 0.25) (layer B.Cu) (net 5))
 (segment (start 137.032999 38.925499) (end 137.032999 40.195499) (width 0.25) (layer B.Cu) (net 5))
 (segment (start 135.89 37.7825) (end 137.032999 38.925499) (width 0.25) (layer B.Cu) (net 5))
 (segment (start 137.16 50.95875) (end 138.58875 52.3875) (width 0.25) (layer B.Cu) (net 5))
 (segment (start 137.16 40.3225) (end 137.16 50.95875) (width 0.25) (layer B.Cu) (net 5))
 (segment (start 137.16 67.6275) (end 137.16 68.8975) (width 0.25) (layer B.Cu) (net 4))
 (segment (start 135.89 66.3575) (end 137.16 67.6275) (width 0.25) (layer B.Cu) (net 4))
 (segment (start 138.58875 63.65875) (end 138.58875 61.9125) (width 0.25) (layer B.Cu) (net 4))
 (segment (start 135.89 66.3575) (end 138.58875 63.65875) (width 0.25) (layer B.Cu) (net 4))
 (segment (start 156.21 67.6275) (end 156.21 68.8975) (width 0.25) (layer B.Cu) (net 2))
 (segment (start 154.94 66.3575) (end 156.21 67.6275) (width 0.25) (layer B.Cu) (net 2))
 (segment (start 157.63875 63.65875) (end 157.63875 61.9125) (width 0.25) (layer B.Cu) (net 2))
 (segment (start 154.94 66.3575) (end 157.63875 63.65875) (width 0.25) (layer B.Cu) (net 2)))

